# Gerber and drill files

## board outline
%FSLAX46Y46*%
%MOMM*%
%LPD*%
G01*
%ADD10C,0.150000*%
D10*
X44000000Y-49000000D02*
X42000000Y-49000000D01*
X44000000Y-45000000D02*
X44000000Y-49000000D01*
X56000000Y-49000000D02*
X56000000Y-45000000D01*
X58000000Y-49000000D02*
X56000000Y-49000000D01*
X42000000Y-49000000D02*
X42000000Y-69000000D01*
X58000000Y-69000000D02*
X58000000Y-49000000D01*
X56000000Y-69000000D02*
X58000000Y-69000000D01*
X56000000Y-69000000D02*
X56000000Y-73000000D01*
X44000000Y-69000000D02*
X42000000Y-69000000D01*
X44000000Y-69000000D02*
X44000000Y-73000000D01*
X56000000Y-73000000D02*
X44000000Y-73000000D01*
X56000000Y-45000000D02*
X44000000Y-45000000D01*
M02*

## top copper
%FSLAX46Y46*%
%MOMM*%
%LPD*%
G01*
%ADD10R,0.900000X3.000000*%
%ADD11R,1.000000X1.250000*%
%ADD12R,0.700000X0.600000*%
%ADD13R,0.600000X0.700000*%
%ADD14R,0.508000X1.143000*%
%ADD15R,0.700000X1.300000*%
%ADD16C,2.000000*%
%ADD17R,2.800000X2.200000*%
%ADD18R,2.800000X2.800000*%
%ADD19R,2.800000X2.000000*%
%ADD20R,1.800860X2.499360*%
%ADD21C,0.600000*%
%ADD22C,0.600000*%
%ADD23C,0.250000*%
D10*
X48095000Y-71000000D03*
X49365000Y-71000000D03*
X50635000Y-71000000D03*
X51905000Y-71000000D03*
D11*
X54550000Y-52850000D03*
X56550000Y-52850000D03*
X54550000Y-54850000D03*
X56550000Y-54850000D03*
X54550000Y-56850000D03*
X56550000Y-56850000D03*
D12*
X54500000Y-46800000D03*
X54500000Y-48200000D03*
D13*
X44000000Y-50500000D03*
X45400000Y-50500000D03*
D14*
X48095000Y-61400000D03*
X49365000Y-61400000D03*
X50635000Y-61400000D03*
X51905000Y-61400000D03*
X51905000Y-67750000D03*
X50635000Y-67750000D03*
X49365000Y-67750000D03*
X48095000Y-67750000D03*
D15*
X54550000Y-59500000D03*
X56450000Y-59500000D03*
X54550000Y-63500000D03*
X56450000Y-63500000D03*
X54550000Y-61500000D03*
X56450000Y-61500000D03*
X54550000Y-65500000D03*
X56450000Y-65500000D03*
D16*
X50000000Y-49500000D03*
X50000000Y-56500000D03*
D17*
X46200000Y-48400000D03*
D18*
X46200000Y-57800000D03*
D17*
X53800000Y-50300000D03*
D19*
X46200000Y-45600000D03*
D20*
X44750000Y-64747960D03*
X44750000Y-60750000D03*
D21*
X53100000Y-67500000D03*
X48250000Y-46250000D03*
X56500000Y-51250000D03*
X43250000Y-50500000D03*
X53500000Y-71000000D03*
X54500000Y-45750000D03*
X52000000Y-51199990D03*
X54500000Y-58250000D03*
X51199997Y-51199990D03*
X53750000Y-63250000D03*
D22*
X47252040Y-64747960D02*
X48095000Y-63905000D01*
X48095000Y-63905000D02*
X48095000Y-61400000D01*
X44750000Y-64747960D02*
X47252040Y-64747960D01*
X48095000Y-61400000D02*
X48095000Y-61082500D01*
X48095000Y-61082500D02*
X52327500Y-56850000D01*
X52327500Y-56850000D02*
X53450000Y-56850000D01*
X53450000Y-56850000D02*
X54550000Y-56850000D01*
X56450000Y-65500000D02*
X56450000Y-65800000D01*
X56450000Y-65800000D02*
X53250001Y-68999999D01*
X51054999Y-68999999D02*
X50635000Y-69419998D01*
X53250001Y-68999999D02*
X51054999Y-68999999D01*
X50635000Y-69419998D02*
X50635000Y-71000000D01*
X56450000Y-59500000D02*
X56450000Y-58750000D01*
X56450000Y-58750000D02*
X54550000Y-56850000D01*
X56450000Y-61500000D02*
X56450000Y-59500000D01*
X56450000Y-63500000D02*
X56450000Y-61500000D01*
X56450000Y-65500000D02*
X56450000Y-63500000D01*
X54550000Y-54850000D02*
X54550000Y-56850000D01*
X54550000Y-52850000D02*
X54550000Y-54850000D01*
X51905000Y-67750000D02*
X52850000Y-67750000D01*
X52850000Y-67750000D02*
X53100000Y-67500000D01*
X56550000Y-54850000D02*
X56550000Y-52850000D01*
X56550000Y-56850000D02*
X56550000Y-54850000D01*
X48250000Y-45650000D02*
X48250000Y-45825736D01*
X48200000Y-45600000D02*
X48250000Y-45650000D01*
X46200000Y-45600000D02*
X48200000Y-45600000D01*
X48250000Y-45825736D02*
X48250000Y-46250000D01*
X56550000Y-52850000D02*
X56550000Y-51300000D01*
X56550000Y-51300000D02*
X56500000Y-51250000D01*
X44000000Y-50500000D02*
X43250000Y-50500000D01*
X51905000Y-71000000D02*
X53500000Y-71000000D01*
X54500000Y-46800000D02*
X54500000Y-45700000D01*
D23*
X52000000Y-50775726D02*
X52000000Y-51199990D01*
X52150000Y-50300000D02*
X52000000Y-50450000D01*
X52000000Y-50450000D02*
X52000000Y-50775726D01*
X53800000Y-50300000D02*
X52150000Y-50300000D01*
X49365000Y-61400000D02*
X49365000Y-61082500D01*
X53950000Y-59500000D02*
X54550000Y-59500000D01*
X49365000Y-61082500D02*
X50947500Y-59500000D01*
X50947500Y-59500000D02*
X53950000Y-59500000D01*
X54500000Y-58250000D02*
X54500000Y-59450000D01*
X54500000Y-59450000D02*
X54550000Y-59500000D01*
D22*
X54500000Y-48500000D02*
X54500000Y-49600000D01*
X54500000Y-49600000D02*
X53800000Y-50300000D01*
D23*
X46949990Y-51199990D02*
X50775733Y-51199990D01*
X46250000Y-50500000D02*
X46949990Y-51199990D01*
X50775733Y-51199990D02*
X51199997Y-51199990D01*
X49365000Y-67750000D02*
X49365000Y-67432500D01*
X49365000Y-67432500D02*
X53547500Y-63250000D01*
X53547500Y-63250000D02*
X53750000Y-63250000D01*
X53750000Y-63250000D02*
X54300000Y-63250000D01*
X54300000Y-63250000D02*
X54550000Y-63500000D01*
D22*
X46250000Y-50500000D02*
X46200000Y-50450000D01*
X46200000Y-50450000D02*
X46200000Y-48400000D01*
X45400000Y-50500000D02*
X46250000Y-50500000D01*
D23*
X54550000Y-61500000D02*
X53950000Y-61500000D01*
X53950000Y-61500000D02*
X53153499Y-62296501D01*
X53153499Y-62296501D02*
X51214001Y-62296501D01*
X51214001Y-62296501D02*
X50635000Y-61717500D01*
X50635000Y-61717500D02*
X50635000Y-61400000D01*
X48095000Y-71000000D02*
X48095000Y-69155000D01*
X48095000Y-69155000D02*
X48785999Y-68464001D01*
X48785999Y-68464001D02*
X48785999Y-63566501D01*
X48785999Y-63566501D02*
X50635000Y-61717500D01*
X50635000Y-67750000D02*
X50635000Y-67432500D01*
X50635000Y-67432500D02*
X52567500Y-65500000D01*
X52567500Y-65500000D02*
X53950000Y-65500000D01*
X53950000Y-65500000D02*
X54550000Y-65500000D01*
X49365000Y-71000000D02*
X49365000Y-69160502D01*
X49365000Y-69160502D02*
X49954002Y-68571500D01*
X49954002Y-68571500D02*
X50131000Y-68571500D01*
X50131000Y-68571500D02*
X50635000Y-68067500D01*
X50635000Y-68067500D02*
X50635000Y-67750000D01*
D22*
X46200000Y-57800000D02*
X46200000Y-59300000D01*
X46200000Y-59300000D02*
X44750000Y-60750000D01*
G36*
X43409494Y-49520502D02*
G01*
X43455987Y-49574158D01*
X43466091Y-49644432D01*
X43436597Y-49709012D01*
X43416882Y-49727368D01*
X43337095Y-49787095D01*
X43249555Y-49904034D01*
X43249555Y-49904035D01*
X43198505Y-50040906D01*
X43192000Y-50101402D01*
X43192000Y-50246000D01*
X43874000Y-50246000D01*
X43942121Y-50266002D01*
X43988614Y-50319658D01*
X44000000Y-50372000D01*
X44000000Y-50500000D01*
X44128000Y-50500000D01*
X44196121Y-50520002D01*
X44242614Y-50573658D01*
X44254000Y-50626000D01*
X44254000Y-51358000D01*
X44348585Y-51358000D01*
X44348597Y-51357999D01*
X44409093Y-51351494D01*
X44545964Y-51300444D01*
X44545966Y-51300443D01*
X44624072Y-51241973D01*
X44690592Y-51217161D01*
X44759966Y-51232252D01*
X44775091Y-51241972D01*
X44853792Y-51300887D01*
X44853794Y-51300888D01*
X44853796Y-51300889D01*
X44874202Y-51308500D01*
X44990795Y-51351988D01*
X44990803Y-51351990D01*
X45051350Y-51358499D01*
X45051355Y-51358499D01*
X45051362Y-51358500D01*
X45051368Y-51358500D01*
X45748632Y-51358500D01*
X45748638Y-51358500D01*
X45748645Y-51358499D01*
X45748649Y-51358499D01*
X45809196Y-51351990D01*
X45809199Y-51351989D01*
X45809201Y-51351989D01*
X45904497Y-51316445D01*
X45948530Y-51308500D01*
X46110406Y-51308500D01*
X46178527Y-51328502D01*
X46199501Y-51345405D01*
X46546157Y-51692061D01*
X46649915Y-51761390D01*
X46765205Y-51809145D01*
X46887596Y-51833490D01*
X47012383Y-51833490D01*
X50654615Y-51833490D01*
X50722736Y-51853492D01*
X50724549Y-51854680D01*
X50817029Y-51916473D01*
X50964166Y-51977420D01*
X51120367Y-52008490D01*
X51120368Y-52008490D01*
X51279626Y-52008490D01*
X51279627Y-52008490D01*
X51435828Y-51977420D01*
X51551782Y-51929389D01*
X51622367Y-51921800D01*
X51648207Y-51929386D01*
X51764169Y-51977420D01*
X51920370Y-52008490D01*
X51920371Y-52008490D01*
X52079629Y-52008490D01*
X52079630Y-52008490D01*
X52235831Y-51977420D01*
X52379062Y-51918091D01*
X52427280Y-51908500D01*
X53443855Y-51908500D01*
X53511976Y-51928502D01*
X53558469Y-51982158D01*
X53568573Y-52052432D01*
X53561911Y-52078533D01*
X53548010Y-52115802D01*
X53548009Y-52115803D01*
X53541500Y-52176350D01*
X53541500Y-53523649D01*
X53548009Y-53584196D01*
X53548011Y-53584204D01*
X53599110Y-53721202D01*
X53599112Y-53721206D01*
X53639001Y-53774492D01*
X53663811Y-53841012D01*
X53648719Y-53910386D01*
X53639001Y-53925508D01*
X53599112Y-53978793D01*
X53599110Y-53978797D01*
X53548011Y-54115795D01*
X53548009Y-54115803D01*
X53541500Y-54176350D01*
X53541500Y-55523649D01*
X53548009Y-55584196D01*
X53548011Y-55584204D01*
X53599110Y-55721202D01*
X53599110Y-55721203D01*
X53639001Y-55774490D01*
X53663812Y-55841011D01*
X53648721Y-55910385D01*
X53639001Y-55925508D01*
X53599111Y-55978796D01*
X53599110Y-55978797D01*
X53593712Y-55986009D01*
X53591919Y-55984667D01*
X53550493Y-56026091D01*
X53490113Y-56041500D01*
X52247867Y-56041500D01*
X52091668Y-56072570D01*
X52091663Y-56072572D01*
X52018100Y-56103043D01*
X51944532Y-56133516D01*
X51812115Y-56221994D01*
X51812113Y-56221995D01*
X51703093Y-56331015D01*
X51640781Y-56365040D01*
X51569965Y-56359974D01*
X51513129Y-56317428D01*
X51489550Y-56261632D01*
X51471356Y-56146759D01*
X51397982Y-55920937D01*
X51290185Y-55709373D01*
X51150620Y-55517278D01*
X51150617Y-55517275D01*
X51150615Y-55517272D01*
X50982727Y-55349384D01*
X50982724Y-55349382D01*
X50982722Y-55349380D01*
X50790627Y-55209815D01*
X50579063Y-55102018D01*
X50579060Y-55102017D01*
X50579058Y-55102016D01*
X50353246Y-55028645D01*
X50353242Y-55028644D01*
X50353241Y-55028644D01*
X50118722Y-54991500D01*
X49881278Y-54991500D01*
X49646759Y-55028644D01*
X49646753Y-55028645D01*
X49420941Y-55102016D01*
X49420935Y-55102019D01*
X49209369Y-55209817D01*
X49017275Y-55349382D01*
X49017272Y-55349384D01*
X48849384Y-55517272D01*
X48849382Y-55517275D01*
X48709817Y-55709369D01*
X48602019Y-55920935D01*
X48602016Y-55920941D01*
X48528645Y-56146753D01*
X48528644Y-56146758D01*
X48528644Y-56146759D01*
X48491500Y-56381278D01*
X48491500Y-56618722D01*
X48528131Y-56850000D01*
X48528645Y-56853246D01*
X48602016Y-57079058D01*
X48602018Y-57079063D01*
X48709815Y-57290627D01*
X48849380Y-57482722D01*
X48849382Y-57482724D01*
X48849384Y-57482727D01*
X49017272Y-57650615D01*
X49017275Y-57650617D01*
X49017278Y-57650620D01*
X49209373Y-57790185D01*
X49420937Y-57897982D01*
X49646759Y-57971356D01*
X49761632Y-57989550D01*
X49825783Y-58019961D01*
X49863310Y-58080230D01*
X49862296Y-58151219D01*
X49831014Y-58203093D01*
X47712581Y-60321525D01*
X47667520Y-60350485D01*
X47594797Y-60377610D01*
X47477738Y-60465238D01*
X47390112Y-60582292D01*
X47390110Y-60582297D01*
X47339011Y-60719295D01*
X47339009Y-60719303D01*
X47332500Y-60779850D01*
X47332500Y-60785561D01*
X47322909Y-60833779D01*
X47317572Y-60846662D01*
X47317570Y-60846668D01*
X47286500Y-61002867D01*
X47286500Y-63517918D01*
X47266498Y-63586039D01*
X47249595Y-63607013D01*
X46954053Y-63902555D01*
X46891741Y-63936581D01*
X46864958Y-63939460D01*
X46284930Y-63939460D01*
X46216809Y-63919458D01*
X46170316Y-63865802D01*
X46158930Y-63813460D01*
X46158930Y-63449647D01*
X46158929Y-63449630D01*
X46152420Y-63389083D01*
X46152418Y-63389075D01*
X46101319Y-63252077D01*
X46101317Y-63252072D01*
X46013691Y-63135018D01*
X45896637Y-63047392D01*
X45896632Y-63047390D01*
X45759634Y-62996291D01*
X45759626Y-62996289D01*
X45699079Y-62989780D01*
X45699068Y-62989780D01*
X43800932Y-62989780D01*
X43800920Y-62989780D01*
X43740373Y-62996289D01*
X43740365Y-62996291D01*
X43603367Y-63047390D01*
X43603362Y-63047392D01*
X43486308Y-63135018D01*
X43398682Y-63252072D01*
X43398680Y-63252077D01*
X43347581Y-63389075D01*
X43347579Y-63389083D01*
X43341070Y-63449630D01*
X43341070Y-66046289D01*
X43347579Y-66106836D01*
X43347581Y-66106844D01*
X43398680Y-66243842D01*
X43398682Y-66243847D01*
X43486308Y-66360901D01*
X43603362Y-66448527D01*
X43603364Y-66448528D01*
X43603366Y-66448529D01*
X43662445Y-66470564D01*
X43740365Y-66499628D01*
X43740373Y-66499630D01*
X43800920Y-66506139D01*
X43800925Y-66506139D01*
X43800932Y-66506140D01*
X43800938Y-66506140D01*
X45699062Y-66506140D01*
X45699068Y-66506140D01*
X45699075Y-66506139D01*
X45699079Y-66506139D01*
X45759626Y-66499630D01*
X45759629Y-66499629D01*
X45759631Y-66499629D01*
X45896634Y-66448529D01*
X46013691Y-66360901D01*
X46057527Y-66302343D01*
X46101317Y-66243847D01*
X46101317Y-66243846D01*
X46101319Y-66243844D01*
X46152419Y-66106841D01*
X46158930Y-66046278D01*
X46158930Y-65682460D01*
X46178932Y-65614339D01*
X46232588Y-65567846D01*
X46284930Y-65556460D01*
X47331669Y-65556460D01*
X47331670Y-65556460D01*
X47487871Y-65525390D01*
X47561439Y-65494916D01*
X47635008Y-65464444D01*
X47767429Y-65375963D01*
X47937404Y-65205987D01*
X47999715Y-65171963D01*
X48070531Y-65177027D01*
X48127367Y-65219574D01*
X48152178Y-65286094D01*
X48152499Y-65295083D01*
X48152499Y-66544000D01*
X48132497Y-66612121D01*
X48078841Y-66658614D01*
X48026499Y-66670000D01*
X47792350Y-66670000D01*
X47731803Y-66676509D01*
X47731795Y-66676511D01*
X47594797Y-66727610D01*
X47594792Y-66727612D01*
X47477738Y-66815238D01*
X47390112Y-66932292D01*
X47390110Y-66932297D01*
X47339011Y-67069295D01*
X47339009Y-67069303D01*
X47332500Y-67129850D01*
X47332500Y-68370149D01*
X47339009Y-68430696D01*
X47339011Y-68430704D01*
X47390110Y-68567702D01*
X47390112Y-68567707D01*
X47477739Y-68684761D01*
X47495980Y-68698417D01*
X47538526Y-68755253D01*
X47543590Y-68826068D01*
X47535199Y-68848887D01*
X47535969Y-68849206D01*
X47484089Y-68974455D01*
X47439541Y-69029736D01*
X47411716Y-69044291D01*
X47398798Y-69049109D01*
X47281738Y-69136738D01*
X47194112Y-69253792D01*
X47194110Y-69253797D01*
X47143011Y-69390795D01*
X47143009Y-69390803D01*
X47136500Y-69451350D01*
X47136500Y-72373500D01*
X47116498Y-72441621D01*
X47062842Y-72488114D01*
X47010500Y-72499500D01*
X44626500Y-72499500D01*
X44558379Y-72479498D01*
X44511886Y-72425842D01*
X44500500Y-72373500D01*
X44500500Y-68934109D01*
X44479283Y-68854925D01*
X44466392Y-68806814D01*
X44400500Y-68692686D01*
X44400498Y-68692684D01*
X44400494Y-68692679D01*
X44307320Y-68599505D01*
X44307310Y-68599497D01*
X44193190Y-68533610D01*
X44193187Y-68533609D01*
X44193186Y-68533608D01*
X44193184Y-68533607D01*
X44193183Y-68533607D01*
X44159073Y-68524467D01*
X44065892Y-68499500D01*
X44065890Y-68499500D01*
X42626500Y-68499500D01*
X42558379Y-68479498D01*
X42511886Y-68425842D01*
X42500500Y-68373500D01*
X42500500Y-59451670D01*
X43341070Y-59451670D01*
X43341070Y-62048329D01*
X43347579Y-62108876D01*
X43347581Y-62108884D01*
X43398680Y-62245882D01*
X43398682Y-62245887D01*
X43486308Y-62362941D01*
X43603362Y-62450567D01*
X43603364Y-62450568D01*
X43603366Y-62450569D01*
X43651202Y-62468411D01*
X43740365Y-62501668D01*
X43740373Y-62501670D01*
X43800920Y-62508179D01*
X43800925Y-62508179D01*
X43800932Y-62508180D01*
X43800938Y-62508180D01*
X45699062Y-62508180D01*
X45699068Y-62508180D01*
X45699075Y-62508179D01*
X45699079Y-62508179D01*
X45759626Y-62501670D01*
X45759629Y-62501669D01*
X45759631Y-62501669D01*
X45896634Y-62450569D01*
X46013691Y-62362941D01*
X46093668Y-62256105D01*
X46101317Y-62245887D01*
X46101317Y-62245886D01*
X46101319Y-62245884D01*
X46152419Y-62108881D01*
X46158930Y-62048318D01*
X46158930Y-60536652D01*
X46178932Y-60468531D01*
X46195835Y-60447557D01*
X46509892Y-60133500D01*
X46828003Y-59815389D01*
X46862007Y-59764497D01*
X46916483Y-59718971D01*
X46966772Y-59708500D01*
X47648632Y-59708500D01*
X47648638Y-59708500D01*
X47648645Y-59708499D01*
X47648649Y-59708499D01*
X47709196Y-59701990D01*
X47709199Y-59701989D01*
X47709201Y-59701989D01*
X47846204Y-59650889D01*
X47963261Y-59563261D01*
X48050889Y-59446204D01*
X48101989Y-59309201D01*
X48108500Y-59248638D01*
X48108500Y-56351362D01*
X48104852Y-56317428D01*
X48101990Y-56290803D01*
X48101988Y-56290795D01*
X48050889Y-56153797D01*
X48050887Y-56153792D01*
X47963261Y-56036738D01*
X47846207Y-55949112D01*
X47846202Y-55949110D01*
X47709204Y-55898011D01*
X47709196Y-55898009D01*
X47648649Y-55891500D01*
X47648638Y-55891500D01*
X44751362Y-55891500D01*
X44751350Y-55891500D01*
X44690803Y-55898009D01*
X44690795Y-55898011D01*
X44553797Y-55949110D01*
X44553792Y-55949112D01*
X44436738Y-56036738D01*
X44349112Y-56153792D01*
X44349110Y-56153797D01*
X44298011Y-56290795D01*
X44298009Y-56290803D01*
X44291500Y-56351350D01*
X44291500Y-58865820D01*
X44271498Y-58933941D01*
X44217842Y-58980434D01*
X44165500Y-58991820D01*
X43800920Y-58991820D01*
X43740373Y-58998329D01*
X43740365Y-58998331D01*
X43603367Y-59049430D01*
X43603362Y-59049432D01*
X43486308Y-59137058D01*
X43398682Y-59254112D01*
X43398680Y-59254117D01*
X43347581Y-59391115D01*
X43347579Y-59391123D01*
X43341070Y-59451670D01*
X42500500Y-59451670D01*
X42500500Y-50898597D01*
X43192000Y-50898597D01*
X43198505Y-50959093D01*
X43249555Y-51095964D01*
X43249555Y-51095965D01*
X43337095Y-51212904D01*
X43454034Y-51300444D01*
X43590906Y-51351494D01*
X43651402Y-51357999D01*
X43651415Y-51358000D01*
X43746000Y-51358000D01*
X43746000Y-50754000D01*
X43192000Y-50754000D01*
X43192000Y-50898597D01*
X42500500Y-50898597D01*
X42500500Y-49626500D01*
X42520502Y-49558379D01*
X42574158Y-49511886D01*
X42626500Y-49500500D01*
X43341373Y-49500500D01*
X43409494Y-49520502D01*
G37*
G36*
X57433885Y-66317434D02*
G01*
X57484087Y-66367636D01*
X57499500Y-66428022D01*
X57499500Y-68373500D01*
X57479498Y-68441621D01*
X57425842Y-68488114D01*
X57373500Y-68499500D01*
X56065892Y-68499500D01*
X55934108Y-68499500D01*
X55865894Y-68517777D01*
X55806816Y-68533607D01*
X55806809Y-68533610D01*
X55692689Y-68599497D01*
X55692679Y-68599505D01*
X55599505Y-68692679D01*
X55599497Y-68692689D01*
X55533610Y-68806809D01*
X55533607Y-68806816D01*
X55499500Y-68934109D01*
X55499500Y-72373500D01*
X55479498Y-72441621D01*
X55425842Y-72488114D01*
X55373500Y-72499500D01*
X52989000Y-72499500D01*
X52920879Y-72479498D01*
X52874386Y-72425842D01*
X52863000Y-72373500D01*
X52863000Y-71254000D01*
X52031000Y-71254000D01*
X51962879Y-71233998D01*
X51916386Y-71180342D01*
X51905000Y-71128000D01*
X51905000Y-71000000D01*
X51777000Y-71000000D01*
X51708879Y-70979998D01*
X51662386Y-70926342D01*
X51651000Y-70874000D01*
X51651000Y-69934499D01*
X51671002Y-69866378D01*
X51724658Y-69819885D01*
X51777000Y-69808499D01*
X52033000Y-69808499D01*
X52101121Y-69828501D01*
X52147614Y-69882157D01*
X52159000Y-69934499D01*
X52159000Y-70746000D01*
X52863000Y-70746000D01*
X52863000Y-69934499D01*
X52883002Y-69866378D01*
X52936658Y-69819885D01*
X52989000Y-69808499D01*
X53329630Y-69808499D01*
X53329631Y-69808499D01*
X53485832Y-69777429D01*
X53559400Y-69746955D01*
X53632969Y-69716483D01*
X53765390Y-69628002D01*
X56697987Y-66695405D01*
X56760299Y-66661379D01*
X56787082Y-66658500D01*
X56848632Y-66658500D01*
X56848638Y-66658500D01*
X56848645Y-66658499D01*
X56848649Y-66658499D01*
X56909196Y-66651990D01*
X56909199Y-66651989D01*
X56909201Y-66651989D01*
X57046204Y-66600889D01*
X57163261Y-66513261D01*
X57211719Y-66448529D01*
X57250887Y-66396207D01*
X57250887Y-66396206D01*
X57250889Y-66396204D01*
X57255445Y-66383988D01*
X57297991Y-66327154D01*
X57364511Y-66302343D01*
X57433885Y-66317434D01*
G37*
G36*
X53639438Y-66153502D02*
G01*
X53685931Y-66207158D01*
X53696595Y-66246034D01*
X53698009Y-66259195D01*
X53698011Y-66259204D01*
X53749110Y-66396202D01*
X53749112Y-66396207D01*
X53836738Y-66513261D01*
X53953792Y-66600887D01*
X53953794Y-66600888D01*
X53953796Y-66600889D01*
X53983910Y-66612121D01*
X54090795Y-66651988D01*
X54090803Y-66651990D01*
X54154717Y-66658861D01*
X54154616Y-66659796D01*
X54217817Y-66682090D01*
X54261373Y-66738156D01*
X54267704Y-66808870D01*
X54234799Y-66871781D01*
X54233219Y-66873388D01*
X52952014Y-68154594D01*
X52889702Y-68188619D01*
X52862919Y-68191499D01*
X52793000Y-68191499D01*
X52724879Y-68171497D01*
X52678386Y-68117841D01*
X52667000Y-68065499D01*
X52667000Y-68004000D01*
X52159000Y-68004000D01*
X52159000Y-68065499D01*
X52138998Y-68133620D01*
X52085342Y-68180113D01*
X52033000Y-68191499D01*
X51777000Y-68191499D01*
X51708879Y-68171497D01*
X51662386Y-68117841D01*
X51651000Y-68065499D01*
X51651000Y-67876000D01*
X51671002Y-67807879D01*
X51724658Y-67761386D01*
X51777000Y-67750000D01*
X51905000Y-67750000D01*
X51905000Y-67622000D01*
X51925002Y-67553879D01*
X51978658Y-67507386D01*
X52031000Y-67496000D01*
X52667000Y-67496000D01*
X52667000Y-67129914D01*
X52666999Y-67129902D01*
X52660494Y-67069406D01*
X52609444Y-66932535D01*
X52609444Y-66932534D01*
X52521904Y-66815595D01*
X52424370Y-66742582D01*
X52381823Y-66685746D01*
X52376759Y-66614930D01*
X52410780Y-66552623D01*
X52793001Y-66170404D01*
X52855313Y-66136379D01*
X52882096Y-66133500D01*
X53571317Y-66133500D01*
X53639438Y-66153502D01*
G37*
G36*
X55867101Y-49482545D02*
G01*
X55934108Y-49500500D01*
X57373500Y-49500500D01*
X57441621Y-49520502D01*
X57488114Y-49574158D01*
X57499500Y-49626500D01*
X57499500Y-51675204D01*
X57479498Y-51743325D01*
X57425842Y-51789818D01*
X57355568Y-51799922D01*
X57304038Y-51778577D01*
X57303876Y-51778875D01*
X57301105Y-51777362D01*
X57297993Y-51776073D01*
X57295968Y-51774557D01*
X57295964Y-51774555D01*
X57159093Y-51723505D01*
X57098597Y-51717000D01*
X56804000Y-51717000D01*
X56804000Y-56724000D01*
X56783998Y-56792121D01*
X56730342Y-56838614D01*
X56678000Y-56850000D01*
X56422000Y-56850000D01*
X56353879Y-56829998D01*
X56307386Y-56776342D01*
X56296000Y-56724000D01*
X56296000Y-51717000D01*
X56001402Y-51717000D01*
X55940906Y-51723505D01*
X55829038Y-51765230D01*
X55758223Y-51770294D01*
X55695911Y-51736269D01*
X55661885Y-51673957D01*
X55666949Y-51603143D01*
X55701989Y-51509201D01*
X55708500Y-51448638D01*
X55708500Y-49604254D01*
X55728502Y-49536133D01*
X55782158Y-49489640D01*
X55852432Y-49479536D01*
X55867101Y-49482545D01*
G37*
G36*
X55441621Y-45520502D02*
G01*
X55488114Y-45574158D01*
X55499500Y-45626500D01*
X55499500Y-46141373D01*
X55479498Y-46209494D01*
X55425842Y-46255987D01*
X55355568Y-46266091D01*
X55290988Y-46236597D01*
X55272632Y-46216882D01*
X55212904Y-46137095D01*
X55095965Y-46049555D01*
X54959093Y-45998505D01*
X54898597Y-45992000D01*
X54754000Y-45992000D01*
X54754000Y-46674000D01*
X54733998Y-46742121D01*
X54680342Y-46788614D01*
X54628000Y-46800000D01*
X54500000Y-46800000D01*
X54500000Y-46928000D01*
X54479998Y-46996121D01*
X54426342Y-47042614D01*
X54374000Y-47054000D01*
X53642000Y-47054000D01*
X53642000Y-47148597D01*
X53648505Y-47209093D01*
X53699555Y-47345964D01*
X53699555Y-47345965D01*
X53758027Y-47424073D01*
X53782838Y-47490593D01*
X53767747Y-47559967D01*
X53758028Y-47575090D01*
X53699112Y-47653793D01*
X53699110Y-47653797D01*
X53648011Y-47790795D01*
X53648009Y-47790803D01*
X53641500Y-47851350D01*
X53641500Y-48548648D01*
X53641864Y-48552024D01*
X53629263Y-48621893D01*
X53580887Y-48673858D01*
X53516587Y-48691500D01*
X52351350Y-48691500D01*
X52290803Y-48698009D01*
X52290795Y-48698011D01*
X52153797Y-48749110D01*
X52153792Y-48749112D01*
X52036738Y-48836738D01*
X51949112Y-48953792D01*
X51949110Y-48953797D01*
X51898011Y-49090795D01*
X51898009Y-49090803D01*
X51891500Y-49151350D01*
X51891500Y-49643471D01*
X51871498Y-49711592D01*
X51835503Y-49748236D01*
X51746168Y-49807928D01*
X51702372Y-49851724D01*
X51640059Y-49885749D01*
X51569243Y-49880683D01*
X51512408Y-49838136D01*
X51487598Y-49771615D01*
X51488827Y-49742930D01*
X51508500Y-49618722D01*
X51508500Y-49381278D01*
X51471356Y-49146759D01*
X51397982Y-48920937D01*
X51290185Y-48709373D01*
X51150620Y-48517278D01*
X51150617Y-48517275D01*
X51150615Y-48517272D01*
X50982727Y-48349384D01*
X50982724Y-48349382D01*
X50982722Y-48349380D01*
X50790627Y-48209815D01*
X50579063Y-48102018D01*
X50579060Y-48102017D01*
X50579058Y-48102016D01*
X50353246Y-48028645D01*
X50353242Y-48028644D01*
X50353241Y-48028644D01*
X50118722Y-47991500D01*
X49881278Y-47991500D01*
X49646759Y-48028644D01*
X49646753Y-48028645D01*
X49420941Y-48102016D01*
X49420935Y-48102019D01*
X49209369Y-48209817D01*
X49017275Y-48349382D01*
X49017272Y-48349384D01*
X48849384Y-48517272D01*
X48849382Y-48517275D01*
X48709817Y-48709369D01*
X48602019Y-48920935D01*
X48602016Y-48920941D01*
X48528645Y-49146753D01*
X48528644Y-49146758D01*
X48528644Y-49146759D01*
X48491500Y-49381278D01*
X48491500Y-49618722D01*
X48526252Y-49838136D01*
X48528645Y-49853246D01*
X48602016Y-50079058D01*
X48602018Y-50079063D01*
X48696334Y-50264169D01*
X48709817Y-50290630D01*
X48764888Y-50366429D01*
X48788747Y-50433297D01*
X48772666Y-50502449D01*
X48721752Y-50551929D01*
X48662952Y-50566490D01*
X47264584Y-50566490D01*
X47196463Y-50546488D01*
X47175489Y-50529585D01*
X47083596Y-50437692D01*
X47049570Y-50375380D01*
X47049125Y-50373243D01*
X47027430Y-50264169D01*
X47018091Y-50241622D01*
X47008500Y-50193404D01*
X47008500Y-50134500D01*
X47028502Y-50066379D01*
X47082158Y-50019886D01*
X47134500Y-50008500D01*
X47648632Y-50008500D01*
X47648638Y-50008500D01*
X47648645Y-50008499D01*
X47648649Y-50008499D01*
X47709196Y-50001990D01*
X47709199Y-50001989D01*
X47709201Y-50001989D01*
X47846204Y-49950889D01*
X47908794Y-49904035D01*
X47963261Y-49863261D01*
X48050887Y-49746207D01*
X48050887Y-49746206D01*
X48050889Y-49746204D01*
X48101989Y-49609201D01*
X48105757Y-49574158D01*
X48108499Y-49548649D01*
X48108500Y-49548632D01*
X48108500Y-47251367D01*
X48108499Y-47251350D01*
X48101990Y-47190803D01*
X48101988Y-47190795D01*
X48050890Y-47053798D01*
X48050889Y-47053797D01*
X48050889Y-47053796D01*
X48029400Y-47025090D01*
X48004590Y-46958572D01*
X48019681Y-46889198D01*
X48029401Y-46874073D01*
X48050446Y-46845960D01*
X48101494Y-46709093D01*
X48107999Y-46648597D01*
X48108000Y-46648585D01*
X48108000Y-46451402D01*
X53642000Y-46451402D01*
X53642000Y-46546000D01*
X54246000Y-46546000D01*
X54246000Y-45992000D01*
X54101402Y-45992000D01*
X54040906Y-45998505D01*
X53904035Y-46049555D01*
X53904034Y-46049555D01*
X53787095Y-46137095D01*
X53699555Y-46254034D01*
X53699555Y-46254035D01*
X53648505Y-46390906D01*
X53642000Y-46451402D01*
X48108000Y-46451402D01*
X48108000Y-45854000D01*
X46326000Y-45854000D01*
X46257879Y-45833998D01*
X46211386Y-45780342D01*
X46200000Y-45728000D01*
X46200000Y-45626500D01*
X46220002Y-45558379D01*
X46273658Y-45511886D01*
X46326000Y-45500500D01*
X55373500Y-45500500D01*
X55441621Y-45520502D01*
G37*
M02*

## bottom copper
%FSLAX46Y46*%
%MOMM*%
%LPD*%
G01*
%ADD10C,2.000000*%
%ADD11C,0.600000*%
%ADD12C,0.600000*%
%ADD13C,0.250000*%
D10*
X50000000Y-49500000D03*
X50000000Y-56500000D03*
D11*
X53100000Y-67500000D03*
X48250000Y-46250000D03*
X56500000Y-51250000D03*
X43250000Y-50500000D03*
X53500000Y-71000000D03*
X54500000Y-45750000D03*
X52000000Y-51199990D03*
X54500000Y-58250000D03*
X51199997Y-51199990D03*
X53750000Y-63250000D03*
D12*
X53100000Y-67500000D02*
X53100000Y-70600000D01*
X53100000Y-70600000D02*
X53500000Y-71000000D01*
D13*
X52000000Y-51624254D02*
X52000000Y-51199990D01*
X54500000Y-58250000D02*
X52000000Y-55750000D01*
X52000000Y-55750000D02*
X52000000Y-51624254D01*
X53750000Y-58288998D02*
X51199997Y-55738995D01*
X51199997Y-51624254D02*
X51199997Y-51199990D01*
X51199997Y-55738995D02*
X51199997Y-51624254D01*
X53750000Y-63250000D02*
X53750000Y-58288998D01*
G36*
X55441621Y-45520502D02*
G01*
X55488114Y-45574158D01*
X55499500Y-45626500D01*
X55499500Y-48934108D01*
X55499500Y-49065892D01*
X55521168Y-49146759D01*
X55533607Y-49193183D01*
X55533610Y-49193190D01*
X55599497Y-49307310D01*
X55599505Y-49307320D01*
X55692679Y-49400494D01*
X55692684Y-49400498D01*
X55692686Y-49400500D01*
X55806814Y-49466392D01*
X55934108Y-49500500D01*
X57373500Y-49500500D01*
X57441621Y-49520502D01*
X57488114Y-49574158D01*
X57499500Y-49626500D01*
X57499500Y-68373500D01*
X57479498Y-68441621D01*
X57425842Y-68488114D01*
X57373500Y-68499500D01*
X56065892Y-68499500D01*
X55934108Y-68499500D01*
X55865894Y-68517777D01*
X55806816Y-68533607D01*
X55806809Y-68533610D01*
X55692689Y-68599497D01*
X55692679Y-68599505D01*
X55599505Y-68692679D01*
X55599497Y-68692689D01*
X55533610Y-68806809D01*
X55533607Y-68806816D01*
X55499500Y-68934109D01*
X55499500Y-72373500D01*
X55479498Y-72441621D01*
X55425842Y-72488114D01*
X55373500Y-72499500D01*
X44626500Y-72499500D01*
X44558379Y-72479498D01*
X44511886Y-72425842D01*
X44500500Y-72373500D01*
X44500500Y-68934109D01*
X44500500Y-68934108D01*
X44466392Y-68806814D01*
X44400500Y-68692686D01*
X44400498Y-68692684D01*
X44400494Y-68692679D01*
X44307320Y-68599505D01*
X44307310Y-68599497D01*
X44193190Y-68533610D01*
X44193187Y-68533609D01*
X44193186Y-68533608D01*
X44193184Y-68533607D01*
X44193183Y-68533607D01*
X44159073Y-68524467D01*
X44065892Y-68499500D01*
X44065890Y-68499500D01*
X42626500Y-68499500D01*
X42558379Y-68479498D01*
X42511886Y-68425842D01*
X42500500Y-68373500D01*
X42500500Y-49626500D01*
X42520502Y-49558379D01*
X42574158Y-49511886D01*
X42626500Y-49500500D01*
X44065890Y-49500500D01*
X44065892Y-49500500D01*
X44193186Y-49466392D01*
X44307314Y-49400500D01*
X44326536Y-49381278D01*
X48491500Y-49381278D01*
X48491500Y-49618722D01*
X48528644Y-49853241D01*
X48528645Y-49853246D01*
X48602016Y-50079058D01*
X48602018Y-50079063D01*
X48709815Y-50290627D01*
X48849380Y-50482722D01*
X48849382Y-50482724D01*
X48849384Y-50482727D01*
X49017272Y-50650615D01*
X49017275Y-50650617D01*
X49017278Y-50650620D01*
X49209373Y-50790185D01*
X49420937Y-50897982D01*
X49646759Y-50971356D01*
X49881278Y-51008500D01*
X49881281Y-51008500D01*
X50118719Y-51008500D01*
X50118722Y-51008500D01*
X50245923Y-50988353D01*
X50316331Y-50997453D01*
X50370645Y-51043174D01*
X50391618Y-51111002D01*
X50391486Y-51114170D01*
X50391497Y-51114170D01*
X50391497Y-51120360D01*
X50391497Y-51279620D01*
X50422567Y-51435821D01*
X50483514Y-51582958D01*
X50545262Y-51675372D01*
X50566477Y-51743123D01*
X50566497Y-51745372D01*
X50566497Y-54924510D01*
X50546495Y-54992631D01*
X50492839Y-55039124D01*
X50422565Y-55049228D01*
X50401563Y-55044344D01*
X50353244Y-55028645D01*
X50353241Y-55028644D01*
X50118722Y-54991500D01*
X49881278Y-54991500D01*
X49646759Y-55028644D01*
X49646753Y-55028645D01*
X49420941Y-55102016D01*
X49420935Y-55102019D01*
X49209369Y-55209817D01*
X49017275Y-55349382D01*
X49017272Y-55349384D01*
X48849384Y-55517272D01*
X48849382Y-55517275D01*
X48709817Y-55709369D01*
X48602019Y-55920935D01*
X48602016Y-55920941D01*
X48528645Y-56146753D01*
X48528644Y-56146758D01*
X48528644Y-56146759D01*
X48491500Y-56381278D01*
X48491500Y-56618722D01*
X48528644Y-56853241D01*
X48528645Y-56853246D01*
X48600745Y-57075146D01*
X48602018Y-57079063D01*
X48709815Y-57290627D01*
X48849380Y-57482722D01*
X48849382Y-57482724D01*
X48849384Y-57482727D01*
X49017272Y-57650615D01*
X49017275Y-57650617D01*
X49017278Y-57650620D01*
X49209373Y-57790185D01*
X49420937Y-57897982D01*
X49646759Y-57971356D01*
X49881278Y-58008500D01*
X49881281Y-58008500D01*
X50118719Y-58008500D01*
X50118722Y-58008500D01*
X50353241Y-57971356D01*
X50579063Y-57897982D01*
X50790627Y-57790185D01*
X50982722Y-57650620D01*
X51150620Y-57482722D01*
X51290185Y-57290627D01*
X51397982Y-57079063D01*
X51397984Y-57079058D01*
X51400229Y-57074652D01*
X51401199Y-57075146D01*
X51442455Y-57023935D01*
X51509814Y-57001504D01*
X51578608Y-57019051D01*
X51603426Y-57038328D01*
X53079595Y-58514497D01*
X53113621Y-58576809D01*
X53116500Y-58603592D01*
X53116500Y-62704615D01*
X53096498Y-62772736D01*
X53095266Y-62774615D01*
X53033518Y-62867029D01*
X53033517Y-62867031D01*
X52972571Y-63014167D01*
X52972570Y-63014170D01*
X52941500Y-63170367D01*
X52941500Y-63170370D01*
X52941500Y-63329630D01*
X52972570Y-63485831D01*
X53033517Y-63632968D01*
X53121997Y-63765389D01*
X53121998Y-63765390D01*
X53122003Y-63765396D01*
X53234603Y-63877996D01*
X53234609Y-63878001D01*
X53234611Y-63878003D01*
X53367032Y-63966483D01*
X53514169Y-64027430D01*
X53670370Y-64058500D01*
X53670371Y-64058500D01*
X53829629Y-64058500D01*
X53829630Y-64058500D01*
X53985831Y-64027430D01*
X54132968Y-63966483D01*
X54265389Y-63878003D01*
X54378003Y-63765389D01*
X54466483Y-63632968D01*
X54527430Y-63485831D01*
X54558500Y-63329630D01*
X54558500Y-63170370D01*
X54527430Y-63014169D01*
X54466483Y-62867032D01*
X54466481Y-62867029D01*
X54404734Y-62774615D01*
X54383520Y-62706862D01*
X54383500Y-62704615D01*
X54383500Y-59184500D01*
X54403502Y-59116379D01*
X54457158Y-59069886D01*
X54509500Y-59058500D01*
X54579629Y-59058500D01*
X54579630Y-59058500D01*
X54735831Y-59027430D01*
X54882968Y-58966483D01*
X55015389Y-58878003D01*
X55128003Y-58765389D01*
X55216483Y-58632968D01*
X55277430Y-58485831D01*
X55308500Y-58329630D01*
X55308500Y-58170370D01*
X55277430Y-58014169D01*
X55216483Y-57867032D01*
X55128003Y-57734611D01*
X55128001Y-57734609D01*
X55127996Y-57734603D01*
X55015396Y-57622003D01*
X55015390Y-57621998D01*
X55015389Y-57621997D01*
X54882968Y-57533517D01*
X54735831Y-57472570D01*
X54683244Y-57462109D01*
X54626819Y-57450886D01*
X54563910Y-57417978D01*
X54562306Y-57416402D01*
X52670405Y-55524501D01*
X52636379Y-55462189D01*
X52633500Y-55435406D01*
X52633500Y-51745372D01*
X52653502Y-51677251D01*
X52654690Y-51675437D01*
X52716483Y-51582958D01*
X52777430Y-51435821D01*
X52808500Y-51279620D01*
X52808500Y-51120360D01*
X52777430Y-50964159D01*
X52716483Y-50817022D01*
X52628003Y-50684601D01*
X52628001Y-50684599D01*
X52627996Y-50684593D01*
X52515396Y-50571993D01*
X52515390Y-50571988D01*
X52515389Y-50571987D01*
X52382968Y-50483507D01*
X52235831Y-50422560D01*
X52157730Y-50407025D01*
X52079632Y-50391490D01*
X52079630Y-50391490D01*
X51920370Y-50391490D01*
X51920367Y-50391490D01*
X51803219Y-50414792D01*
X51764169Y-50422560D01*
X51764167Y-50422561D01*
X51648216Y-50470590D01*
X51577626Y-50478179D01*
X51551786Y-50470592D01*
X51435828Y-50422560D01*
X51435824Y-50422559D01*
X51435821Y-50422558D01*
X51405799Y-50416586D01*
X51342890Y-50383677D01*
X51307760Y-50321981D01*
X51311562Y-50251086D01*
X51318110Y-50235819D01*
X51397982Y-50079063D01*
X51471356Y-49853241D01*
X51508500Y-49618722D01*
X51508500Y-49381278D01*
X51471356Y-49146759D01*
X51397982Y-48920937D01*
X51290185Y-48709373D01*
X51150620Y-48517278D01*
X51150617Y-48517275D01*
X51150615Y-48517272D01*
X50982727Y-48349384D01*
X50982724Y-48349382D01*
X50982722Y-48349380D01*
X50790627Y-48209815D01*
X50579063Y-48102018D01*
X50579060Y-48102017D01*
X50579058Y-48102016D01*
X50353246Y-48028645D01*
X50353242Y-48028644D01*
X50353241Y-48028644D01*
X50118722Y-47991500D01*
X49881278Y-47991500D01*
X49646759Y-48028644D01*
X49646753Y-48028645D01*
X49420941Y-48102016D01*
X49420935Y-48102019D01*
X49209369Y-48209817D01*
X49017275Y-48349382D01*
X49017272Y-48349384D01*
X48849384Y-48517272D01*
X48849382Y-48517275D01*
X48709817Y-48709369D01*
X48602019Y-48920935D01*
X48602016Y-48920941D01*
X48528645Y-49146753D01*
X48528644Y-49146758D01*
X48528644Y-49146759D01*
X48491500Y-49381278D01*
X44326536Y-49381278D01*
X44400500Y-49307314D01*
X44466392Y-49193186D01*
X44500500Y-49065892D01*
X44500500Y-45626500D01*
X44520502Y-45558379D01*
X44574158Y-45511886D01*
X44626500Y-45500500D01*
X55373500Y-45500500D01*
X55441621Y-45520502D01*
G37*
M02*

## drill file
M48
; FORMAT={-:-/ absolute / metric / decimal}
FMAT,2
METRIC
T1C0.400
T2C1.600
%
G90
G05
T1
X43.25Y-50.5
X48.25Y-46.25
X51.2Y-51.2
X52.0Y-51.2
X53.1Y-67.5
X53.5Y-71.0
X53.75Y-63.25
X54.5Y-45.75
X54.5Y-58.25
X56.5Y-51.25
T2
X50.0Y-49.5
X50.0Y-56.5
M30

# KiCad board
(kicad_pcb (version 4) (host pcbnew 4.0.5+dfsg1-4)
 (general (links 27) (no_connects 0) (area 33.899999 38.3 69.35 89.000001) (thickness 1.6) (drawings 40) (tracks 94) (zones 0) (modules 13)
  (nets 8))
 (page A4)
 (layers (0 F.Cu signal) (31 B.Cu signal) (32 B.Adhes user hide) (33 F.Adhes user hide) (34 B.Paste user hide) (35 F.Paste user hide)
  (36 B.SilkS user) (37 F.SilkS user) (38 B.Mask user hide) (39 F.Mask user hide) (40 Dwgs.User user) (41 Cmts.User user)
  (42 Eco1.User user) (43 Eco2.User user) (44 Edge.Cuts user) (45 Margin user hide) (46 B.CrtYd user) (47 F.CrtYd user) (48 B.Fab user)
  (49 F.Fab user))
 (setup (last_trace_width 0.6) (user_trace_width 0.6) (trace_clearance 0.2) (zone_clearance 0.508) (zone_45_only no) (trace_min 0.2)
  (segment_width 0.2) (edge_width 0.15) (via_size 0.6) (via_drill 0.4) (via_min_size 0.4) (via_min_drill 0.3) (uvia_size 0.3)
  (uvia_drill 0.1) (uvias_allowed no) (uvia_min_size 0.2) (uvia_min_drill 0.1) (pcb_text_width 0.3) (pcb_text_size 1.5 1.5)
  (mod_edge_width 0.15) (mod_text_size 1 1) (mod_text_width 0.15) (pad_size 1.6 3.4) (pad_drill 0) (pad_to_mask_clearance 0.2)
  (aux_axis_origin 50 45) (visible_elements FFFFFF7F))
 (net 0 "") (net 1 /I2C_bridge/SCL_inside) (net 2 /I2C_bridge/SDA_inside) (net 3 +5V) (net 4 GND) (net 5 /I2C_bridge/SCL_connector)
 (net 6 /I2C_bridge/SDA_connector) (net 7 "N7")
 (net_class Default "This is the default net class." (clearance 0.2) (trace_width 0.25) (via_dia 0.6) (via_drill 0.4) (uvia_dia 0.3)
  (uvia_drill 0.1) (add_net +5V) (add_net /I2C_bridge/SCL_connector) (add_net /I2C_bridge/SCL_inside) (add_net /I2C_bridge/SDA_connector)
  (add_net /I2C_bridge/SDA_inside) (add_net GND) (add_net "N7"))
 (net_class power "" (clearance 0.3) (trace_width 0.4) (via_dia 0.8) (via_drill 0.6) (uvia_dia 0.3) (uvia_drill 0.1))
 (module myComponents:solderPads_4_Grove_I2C (layer F.Cu) (at 50 71)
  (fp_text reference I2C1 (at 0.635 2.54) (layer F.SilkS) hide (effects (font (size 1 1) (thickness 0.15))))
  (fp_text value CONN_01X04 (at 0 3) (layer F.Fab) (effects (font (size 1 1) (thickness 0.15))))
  (pad 1 smd rect (at -1.905 0) (size 0.9 3) (layers F.Cu F.Paste F.Mask) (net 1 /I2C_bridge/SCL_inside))
  (pad 2 smd rect (at -0.635 0) (size 0.9 3) (layers F.Cu F.Paste F.Mask) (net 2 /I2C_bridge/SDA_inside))
  (pad 3 smd rect (at 0.635 0) (size 0.9 3) (layers F.Cu F.Paste F.Mask) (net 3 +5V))
  (pad 4 smd rect (at 1.905 0) (size 0.9 3) (layers F.Cu F.Paste F.Mask) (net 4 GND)))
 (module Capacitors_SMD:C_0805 (layer F.Cu) (at 55.55 52.85)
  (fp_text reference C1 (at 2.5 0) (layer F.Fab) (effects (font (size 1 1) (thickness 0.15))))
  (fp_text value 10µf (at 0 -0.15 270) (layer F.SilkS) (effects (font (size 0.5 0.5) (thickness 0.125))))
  (pad 1 smd rect (at -1 0) (size 1 1.25) (layers F.Cu F.Paste F.Mask) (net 3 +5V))
  (pad 2 smd rect (at 1 0) (size 1 1.25) (layers F.Cu F.Paste F.Mask) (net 4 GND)))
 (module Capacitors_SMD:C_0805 (layer F.Cu) (at 55.55 54.85)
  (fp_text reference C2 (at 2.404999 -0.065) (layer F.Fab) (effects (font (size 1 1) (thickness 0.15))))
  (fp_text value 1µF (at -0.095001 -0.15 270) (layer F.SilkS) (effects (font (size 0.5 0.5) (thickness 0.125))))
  (pad 1 smd rect (at -1 0) (size 1 1.25) (layers F.Cu F.Paste F.Mask) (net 3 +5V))
  (pad 2 smd rect (at 1 0) (size 1 1.25) (layers F.Cu F.Paste F.Mask) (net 4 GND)))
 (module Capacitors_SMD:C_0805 (layer F.Cu) (at 55.55 56.85)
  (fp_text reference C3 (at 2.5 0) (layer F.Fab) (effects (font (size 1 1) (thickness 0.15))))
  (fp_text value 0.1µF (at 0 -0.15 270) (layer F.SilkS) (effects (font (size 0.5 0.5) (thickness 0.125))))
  (pad 1 smd rect (at -1 0) (size 1 1.25) (layers F.Cu F.Paste F.Mask) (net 3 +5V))
  (pad 2 smd rect (at 1 0) (size 1 1.25) (layers F.Cu F.Paste F.Mask) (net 4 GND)))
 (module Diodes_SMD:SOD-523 (layer F.Cu) (at 54.5 47.5 90)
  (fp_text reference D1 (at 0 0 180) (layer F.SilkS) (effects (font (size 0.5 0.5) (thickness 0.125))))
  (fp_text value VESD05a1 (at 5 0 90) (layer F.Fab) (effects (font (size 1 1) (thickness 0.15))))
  (pad 2 smd rect (at 0.7 0 270) (size 0.6 0.7) (layers F.Cu F.Paste F.Mask) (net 4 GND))
  (pad 1 smd rect (at -0.7 0 270) (size 0.6 0.7) (layers F.Cu F.Paste F.Mask) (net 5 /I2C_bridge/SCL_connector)))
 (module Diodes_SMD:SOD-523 (layer F.Cu) (at 44.7 50.5 180)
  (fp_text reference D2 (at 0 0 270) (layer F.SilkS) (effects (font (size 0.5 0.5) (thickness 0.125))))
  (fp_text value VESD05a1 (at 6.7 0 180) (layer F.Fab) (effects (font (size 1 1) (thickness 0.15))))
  (pad 2 smd rect (at 0.7 0) (size 0.6 0.7) (layers F.Cu F.Paste F.Mask) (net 4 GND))
  (pad 1 smd rect (at -0.7 0) (size 0.6 0.7) (layers F.Cu F.Paste F.Mask) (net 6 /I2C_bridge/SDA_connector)))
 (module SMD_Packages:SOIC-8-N (layer F.Cu) (at 50 64.575)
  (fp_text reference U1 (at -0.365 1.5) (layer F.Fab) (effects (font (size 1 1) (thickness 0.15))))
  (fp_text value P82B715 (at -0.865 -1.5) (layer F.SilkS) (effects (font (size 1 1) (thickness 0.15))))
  (pad 8 smd rect (at -1.905 -3.175) (size 0.508 1.143) (layers F.Cu F.Paste F.Mask) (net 3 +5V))
  (pad 7 smd rect (at -0.635 -3.175) (size 0.508 1.143) (layers F.Cu F.Paste F.Mask) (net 5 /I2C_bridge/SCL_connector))
  (pad 6 smd rect (at 0.635 -3.175) (size 0.508 1.143) (layers F.Cu F.Paste F.Mask) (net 1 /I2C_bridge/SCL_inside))
  (pad 5 smd rect (at 1.905 -3.175) (size 0.508 1.143) (layers F.Cu F.Paste F.Mask))
  (pad 4 smd rect (at 1.905 3.175) (size 0.508 1.143) (layers F.Cu F.Paste F.Mask) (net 4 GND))
  (pad 3 smd rect (at 0.635 3.175) (size 0.508 1.143) (layers F.Cu F.Paste F.Mask) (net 2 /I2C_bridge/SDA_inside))
  (pad 2 smd rect (at -0.635 3.175) (size 0.508 1.143) (layers F.Cu F.Paste F.Mask) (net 6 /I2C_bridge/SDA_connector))
  (pad 1 smd rect (at -1.905 3.175) (size 0.508 1.143) (layers F.Cu F.Paste F.Mask)))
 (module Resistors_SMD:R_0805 (layer F.Cu) (at 55.5 59.5)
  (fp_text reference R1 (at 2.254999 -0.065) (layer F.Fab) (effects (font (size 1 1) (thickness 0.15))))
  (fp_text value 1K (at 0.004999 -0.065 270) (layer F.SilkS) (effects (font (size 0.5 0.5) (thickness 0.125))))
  (pad 1 smd rect (at -0.95 0) (size 0.7 1.3) (layers F.Cu F.Paste F.Mask) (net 5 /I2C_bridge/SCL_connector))
  (pad 2 smd rect (at 0.95 0) (size 0.7 1.3) (layers F.Cu F.Paste F.Mask) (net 3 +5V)))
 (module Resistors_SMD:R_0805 (layer F.Cu) (at 55.5 63.5)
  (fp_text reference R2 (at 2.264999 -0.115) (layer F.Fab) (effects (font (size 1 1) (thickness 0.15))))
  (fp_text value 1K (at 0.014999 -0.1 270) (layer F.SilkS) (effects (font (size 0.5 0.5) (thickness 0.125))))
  (pad 1 smd rect (at -0.95 0) (size 0.7 1.3) (layers F.Cu F.Paste F.Mask) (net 6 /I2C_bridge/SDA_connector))
  (pad 2 smd rect (at 0.95 0) (size 0.7 1.3) (layers F.Cu F.Paste F.Mask) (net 3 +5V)))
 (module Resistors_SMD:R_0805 (layer F.Cu) (at 55.5 61.5)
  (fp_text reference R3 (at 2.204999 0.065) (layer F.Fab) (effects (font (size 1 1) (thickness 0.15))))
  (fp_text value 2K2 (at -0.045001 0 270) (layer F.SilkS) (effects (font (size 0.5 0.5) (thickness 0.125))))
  (pad 1 smd rect (at -0.95 0) (size 0.7 1.3) (layers F.Cu F.Paste F.Mask) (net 1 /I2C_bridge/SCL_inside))
  (pad 2 smd rect (at 0.95 0) (size 0.7 1.3) (layers F.Cu F.Paste F.Mask) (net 3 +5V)))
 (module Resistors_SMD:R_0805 (layer F.Cu) (at 55.5 65.5)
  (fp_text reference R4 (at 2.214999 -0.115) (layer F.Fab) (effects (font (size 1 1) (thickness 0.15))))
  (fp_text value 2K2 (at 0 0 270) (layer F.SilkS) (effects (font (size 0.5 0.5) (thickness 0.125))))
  (pad 1 smd rect (at -0.95 0) (size 0.7 1.3) (layers F.Cu F.Paste F.Mask) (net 2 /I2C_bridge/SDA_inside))
  (pad 2 smd rect (at 0.95 0) (size 0.7 1.3) (layers F.Cu F.Paste F.Mask) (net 3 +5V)))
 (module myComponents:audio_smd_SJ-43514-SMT (layer F.Cu) (at 50 45 270)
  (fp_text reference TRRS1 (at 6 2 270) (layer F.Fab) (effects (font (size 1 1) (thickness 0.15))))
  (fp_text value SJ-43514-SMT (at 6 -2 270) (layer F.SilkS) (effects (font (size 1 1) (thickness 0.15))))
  (pad "" thru_hole circle (at 4.5 0 270) (size 2 2) (drill 1.6) (layers *.Cu *.Mask F.SilkS))
  (pad "" thru_hole circle (at 11.5 0 270) (size 2 2) (drill 1.6) (layers *.Cu *.Mask F.SilkS))
  (pad 4 smd rect (at 3.4 3.8 270) (size 2.2 2.8) (layers F.Cu F.Paste F.Mask) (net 6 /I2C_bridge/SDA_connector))
  (pad 2 smd rect (at 12.8 3.8 270) (size 2.8 2.8) (layers F.Cu F.Paste F.Mask) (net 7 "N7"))
  (pad 3 smd rect (at 5.3 -3.8 270) (size 2.2 2.8) (layers F.Cu F.Paste F.Mask) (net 5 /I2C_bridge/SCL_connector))
  (pad 1 smd rect (at 0.6 3.8 270) (size 2 2.8) (layers F.Cu F.Paste F.Mask) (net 4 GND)))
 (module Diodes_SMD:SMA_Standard (layer F.Cu) (at 44.75 62.74898 90)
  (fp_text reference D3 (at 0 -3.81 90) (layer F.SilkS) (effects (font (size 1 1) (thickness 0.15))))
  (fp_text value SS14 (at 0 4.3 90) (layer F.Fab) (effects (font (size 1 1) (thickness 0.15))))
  (pad 1 smd rect (at -1.99898 0 90) (size 2.49936 1.80086) (layers F.Cu F.Paste F.Mask) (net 3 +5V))
  (pad 2 smd rect (at 1.99898 0 90) (size 2.49936 1.80086) (layers F.Cu F.Paste F.Mask) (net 7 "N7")))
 (gr_line (start 44 49) (end 42 49) (layer Edge.Cuts) (width 0.15))
 (gr_line (start 44 45) (end 44 49) (layer Edge.Cuts) (width 0.15))
 (gr_line (start 56 49) (end 56 45) (layer Edge.Cuts) (width 0.15))
 (gr_line (start 58 49) (end 56 49) (layer Edge.Cuts) (width 0.15))
 (gr_line (start 42 49) (end 42 69) (layer Edge.Cuts) (width 0.15))
 (gr_line (start 58 69) (end 58 49) (layer Edge.Cuts) (width 0.15))
 (gr_line (start 56 69) (end 58 69) (layer Edge.Cuts) (width 0.15))
 (gr_line (start 56 69) (end 56 73) (layer Edge.Cuts) (width 0.15))
 (gr_line (start 44 69) (end 42 69) (layer Edge.Cuts) (width 0.15))
 (gr_line (start 44 69) (end 44 73) (layer Edge.Cuts) (width 0.15))
 (gr_line (start 56 73) (end 44 73) (layer Edge.Cuts) (width 0.15))
 (gr_line (start 56 45) (end 44 45) (layer Edge.Cuts) (width 0.15))
 (segment (start 47.25204 64.74796) (end 48.095 63.905) (width 0.6) (layer F.Cu) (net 3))
 (segment (start 48.095 63.905) (end 48.095 61.4) (width 0.6) (layer F.Cu) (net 3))
 (segment (start 44.75 64.74796) (end 47.25204 64.74796) (width 0.6) (layer F.Cu) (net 3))
 (segment (start 48.095 61.4) (end 48.095 61.0825) (width 0.6) (layer F.Cu) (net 3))
 (segment (start 48.095 61.0825) (end 52.3275 56.85) (width 0.6) (layer F.Cu) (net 3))
 (segment (start 52.3275 56.85) (end 53.45 56.85) (width 0.6) (layer F.Cu) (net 3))
 (segment (start 53.45 56.85) (end 54.55 56.85) (width 0.6) (layer F.Cu) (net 3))
 (segment (start 56.45 65.5) (end 56.45 65.8) (width 0.6) (layer F.Cu) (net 3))
 (segment (start 56.45 65.8) (end 53.250001 68.999999) (width 0.6) (layer F.Cu) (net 3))
 (segment (start 51.054999 68.999999) (end 50.635 69.419998) (width 0.6) (layer F.Cu) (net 3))
 (segment (start 53.250001 68.999999) (end 51.054999 68.999999) (width 0.6) (layer F.Cu) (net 3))
 (segment (start 50.635 69.419998) (end 50.635 71) (width 0.6) (layer F.Cu) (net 3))
 (segment (start 56.45 59.5) (end 56.45 58.75) (width 0.6) (layer F.Cu) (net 3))
 (segment (start 56.45 58.75) (end 54.55 56.85) (width 0.6) (layer F.Cu) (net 3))
 (segment (start 56.45 61.5) (end 56.45 59.5) (width 0.6) (layer F.Cu) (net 3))
 (segment (start 56.45 63.5) (end 56.45 61.5) (width 0.6) (layer F.Cu) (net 3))
 (segment (start 56.45 65.5) (end 56.45 63.5) (width 0.6) (layer F.Cu) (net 3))
 (segment (start 54.55 54.85) (end 54.55 56.85) (width 0.6) (layer F.Cu) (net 3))
 (segment (start 54.55 52.85) (end 54.55 54.85) (width 0.6) (layer F.Cu) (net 3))
 (segment (start 53.1 67.5) (end 53.1 70.6) (width 0.6) (layer B.Cu) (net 4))
 (segment (start 53.1 70.6) (end 53.5 71) (width 0.6) (layer B.Cu) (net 4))
 (segment (start 51.905 67.75) (end 52.85 67.75) (width 0.6) (layer F.Cu) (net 4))
 (segment (start 52.85 67.75) (end 53.1 67.5) (width 0.6) (layer F.Cu) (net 4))
 (via (at 53.1 67.5) (size 0.6) (drill 0.4) (layers F.Cu B.Cu) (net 4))
 (segment (start 56.55 54.85) (end 56.55 52.85) (width 0.6) (layer F.Cu) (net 4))
 (segment (start 56.55 56.85) (end 56.55 54.85) (width 0.6) (layer F.Cu) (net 4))
 (segment (start 48.25 45.65) (end 48.25 45.825736) (width 0.6) (layer F.Cu) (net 4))
 (segment (start 48.2 45.6) (end 48.25 45.65) (width 0.6) (layer F.Cu) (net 4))
 (segment (start 46.2 45.6) (end 48.2 45.6) (width 0.6) (layer F.Cu) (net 4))
 (segment (start 48.25 45.825736) (end 48.25 46.25) (width 0.6) (layer F.Cu) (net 4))
 (via (at 48.25 46.25) (size 0.6) (drill 0.4) (layers F.Cu B.Cu) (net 4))
 (segment (start 56.55 52.85) (end 56.55 51.3) (width 0.6) (layer F.Cu) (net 4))
 (segment (start 56.55 51.3) (end 56.5 51.25) (width 0.6) (layer F.Cu) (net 4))
 (via (at 56.5 51.25) (size 0.6) (drill 0.4) (layers F.Cu B.Cu) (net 4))
 (segment (start 44 50.5) (end 43.25 50.5) (width 0.6) (layer F.Cu) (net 4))
 (via (at 43.25 50.5) (size 0.6) (drill 0.4) (layers F.Cu B.Cu) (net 4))
 (segment (start 51.905 71) (end 53.5 71) (width 0.6) (layer F.Cu) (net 4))
 (via (at 53.5 71) (size 0.6) (drill 0.4) (layers F.Cu B.Cu) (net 4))
 (segment (start 54.5 46.8) (end 54.5 45.7) (width 0.6) (layer F.Cu) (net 4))
 (via (at 54.5 45.75) (size 0.6) (drill 0.4) (layers F.Cu B.Cu) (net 4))
 (segment (start 52 50.775726) (end 52 51.19999) (width 0.25) (layer F.Cu) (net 5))
 (segment (start 52.15 50.3) (end 52 50.45) (width 0.25) (layer F.Cu) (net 5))
 (segment (start 52 50.45) (end 52 50.775726) (width 0.25) (layer F.Cu) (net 5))
 (via (at 52 51.19999) (size 0.6) (drill 0.4) (layers F.Cu B.Cu) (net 5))
 (segment (start 52 51.624254) (end 52 51.19999) (width 0.25) (layer B.Cu) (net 5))
 (segment (start 54.5 58.25) (end 52 55.75) (width 0.25) (layer B.Cu) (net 5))
 (segment (start 52 55.75) (end 52 51.624254) (width 0.25) (layer B.Cu) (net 5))
 (segment (start 53.8 50.3) (end 52.15 50.3) (width 0.25) (layer F.Cu) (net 5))
 (segment (start 49.365 61.4) (end 49.365 61.0825) (width 0.25) (layer F.Cu) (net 5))
 (segment (start 53.95 59.5) (end 54.55 59.5) (width 0.25) (layer F.Cu) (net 5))
 (segment (start 49.365 61.0825) (end 50.9475 59.5) (width 0.25) (layer F.Cu) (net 5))
 (segment (start 50.9475 59.5) (end 53.95 59.5) (width 0.25) (layer F.Cu) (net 5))
 (segment (start 54.5 58.25) (end 54.5 59.45) (width 0.25) (layer F.Cu) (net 5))
 (segment (start 54.5 59.45) (end 54.55 59.5) (width 0.25) (layer F.Cu) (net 5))
 (via (at 54.5 58.25) (size 0.6) (drill 0.4) (layers F.Cu B.Cu) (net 5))
 (segment (start 54.5 48.5) (end 54.5 49.6) (width 0.6) (layer F.Cu) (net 5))
 (segment (start 54.5 49.6) (end 53.8 50.3) (width 0.6) (layer F.Cu) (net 5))
 (segment (start 53.75 58.288998) (end 51.199997 55.738995) (width 0.25) (layer B.Cu) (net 6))
 (segment (start 46.94999 51.19999) (end 50.775733 51.19999) (width 0.25) (layer F.Cu) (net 6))
 (segment (start 46.25 50.5) (end 46.94999 51.19999) (width 0.25) (layer F.Cu) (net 6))
 (segment (start 51.199997 51.624254) (end 51.199997 51.19999) (width 0.25) (layer B.Cu) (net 6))
 (segment (start 51.199997 55.738995) (end 51.199997 51.624254) (width 0.25) (layer B.Cu) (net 6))
 (segment (start 50.775733 51.19999) (end 51.199997 51.19999) (width 0.25) (layer F.Cu) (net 6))
 (segment (start 53.75 63.25) (end 53.75 58.288998) (width 0.25) (layer B.Cu) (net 6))
 (via (at 51.199997 51.19999) (size 0.6) (drill 0.4) (layers F.Cu B.Cu) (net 6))
 (segment (start 49.365 67.75) (end 49.365 67.4325) (width 0.25) (layer F.Cu) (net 6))
 (segment (start 49.365 67.4325) (end 53.5475 63.25) (width 0.25) (layer F.Cu) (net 6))
 (segment (start 53.5475 63.25) (end 53.75 63.25) (width 0.25) (layer F.Cu) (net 6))
 (segment (start 53.75 63.25) (end 54.3 63.25) (width 0.25) (layer F.Cu) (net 6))
 (segment (start 54.3 63.25) (end 54.55 63.5) (width 0.25) (layer F.Cu) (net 6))
 (via (at 53.75 63.25) (size 0.6) (drill 0.4) (layers F.Cu B.Cu) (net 6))
 (segment (start 46.25 50.5) (end 46.2 50.45) (width 0.6) (layer F.Cu) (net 6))
 (segment (start 46.2 50.45) (end 46.2 48.4) (width 0.6) (layer F.Cu) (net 6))
 (segment (start 45.4 50.5) (end 46.25 50.5) (width 0.6) (layer F.Cu) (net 6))
 (segment (start 54.55 61.5) (end 53.95 61.5) (width 0.25) (layer F.Cu) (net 1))
 (segment (start 53.95 61.5) (end 53.153499 62.296501) (width 0.25) (layer F.Cu) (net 1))
 (segment (start 53.153499 62.296501) (end 51.214001 62.296501) (width 0.25) (layer F.Cu) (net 1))
 (segment (start 51.214001 62.296501) (end 50.635 61.7175) (width 0.25) (layer F.Cu) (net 1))
 (segment (start 50.635 61.7175) (end 50.635 61.4) (width 0.25) (layer F.Cu) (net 1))
 (segment (start 48.095 71) (end 48.095 69.155) (width 0.25) (layer F.Cu) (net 1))
 (segment (start 48.095 69.155) (end 48.785999 68.464001) (width 0.25) (layer F.Cu) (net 1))
 (segment (start 48.785999 68.464001) (end 48.785999 63.566501) (width 0.25) (layer F.Cu) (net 1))
 (segment (start 48.785999 63.566501) (end 50.635 61.7175) (width 0.25) (layer F.Cu) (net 1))
 (segment (start 50.635 67.75) (end 50.635 67.4325) (width 0.25) (layer F.Cu) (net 2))
 (segment (start 50.635 67.4325) (end 52.5675 65.5) (width 0.25) (layer F.Cu) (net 2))
 (segment (start 52.5675 65.5) (end 53.95 65.5) (width 0.25) (layer F.Cu) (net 2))
 (segment (start 53.95 65.5) (end 54.55 65.5) (width 0.25) (layer F.Cu) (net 2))
 (segment (start 49.365 71) (end 49.365 69.160502) (width 0.25) (layer F.Cu) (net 2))
 (segment (start 49.365 69.160502) (end 49.954002 68.5715) (width 0.25) (layer F.Cu) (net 2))
 (segment (start 49.954002 68.5715) (end 50.131 68.5715) (width 0.25) (layer F.Cu) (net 2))
 (segment (start 50.131 68.5715) (end 50.635 68.0675) (width 0.25) (layer F.Cu) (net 2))
 (segment (start 50.635 68.0675) (end 50.635 67.75) (width 0.25) (layer F.Cu) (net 2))
 (segment (start 46.2 57.8) (end 46.2 59.3) (width 0.6) (layer F.Cu) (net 7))
 (segment (start 46.2 59.3) (end 44.75 60.75) (width 0.6) (layer F.Cu) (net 7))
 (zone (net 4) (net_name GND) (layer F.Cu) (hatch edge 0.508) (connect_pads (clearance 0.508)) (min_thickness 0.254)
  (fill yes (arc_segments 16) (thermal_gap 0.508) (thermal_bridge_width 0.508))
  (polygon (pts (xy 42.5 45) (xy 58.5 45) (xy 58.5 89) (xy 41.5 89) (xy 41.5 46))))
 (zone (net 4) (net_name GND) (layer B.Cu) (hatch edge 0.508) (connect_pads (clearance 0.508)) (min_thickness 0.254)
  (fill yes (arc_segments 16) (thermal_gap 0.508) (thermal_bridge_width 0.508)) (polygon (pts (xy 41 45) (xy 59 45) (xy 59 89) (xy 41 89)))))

